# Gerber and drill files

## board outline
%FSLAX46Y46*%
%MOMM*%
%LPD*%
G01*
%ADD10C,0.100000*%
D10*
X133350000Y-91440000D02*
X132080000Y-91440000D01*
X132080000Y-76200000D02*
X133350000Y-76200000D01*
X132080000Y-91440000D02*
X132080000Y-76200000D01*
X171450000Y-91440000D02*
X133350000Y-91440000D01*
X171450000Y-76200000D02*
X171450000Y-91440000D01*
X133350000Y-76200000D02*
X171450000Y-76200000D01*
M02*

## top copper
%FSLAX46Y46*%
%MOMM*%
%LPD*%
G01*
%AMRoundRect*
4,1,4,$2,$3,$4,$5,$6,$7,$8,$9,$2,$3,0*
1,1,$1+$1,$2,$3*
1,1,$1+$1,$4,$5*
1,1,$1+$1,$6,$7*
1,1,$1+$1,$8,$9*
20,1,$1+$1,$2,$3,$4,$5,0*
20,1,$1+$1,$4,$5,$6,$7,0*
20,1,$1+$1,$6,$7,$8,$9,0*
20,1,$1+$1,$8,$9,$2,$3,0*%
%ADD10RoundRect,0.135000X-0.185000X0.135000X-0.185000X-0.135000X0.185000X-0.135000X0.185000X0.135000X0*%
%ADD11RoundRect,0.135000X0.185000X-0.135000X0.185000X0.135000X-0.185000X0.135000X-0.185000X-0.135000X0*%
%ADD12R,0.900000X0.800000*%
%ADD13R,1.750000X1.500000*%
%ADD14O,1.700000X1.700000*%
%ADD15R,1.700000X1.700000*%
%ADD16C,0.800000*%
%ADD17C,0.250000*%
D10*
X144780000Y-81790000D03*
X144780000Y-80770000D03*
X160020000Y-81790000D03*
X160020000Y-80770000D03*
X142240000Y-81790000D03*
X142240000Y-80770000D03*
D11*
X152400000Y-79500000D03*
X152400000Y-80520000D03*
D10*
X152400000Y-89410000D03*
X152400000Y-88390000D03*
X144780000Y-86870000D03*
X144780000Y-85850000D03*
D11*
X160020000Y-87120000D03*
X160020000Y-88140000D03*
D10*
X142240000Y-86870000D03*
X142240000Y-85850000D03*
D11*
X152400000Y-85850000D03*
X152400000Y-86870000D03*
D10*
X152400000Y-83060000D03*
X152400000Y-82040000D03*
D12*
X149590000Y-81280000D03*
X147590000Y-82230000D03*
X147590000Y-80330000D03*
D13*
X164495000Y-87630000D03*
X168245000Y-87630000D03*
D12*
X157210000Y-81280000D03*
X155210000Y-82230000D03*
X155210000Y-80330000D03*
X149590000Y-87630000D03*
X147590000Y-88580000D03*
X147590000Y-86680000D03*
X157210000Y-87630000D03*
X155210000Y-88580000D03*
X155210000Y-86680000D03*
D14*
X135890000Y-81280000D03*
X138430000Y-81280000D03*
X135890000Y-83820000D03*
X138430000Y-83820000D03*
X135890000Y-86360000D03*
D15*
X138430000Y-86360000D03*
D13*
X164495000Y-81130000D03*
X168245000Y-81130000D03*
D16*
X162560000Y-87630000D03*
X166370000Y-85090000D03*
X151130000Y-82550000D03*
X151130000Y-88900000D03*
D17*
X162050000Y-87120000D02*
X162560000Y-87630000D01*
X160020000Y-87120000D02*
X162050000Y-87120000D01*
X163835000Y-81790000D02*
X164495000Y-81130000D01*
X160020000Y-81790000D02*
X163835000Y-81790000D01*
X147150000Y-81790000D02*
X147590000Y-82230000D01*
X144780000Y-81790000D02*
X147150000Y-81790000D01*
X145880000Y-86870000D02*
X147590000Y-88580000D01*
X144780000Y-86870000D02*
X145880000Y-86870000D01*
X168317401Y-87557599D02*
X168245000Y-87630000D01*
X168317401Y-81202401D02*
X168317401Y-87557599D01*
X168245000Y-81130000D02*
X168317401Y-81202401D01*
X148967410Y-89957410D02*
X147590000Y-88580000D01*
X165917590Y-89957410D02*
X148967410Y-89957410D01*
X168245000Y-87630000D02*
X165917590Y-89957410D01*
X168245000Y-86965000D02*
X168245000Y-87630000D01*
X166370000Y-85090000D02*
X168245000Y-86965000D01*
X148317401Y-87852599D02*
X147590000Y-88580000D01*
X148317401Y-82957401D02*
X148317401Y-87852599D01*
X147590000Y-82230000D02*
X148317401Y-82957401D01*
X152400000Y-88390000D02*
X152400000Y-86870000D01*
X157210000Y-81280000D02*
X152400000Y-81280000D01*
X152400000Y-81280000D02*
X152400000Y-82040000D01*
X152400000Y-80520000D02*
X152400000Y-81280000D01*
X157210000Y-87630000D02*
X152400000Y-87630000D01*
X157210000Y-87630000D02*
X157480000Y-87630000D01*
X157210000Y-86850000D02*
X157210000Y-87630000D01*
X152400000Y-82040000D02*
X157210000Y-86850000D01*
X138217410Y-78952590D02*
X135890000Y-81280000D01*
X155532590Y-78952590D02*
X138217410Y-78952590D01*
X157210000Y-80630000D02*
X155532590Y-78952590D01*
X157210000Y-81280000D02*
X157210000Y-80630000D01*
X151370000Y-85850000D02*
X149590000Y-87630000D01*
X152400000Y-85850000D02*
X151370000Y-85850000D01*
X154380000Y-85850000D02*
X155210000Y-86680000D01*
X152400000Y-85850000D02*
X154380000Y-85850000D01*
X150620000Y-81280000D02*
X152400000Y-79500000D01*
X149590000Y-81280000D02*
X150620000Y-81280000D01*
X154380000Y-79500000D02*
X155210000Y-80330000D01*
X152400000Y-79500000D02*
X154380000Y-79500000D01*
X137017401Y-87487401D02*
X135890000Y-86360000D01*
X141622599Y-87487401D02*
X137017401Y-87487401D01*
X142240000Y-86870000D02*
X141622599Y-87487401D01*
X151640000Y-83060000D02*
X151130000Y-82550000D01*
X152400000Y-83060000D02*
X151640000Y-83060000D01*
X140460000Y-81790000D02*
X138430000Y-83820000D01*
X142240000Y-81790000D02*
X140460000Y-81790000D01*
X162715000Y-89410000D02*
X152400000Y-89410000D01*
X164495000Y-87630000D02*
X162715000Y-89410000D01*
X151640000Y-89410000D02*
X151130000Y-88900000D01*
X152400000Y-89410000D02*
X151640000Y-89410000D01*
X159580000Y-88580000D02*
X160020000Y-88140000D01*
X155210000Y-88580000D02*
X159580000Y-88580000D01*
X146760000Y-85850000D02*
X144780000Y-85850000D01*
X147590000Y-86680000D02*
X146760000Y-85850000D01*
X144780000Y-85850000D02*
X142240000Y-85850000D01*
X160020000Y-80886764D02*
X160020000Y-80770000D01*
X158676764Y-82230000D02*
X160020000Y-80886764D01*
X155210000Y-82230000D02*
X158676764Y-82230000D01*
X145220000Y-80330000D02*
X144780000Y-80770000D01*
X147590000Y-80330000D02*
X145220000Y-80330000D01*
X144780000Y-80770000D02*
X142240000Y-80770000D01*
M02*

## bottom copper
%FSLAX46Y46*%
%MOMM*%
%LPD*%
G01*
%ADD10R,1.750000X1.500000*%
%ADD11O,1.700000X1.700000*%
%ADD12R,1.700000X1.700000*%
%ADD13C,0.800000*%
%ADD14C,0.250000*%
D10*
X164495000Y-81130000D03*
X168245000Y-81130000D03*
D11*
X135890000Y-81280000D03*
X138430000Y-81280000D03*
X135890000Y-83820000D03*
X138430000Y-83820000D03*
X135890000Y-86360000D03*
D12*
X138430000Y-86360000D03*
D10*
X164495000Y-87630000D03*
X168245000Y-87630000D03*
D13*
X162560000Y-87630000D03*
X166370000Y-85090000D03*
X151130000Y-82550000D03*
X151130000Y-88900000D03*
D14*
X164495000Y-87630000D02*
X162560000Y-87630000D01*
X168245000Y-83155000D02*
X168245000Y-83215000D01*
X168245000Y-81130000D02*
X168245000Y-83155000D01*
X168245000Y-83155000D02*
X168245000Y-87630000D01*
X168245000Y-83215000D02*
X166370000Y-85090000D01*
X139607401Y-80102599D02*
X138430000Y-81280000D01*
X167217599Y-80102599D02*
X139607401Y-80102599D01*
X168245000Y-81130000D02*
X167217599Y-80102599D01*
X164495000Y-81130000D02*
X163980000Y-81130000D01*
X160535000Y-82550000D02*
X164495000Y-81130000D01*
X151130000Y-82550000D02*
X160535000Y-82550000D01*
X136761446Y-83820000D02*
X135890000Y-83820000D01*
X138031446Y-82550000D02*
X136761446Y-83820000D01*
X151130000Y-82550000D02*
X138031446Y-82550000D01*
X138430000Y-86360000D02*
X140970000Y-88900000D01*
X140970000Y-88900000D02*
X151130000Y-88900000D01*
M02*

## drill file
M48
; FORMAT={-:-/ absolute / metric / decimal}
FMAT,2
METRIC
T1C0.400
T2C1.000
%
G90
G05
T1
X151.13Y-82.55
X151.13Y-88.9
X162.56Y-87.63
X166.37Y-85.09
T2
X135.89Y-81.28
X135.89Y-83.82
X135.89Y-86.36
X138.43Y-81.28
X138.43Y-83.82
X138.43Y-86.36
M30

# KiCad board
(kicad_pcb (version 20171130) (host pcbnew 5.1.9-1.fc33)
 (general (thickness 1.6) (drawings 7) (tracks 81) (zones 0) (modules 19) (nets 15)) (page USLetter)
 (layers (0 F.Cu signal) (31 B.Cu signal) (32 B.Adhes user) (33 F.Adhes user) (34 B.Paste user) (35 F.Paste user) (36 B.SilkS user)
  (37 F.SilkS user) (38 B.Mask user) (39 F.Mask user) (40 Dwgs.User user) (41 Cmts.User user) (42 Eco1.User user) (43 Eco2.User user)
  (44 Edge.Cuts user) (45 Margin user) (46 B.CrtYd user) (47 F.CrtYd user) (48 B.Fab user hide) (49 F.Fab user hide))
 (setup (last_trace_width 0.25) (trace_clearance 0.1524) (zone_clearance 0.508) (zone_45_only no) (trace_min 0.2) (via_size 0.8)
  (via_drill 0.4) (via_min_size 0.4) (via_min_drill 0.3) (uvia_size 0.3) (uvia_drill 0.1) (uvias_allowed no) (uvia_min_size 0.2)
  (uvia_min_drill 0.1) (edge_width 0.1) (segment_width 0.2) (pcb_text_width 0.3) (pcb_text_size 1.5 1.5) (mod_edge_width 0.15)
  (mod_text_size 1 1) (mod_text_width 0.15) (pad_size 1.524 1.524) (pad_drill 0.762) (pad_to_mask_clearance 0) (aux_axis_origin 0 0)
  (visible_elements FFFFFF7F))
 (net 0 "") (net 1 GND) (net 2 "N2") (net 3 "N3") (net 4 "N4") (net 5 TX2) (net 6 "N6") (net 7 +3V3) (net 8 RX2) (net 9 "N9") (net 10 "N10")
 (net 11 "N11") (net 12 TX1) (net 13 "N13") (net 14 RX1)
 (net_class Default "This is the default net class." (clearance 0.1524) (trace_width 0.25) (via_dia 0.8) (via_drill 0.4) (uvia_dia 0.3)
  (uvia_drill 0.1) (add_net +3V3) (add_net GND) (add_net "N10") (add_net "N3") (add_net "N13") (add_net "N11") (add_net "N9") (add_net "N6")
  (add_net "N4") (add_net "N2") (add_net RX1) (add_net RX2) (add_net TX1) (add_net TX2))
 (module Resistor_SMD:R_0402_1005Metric (layer F.Cu) (at 144.78 81.28 270)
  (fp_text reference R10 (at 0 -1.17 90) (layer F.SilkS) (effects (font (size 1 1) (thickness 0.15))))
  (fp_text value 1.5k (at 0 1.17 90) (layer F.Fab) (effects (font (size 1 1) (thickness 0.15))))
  (pad 2 smd roundrect (at 0.51 0 270) (size 0.54 0.64) (layers F.Cu F.Paste F.Mask) (roundrect_rratio 0.25) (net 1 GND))
  (pad 1 smd roundrect (at -0.51 0 270) (size 0.54 0.64) (layers F.Cu F.Paste F.Mask) (roundrect_rratio 0.25) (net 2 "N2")))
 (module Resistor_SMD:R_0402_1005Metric (layer F.Cu) (at 160.02 81.28 270)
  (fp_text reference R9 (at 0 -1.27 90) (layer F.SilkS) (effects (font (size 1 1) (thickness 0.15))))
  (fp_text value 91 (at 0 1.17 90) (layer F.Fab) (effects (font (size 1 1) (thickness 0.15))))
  (pad 2 smd roundrect (at 0.51 0 270) (size 0.54 0.64) (layers F.Cu F.Paste F.Mask) (roundrect_rratio 0.25) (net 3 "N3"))
  (pad 1 smd roundrect (at -0.51 0 270) (size 0.54 0.64) (layers F.Cu F.Paste F.Mask) (roundrect_rratio 0.25) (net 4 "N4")))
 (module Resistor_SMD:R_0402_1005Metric (layer F.Cu) (at 142.24 81.28 270)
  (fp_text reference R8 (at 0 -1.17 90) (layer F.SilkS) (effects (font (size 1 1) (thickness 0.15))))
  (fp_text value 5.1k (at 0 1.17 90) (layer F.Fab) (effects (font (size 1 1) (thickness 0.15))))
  (pad 2 smd roundrect (at 0.51 0 270) (size 0.54 0.64) (layers F.Cu F.Paste F.Mask) (roundrect_rratio 0.25) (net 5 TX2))
  (pad 1 smd roundrect (at -0.51 0 270) (size 0.54 0.64) (layers F.Cu F.Paste F.Mask) (roundrect_rratio 0.25) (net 2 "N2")))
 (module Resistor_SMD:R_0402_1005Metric (layer F.Cu) (at 152.4 80.01 90)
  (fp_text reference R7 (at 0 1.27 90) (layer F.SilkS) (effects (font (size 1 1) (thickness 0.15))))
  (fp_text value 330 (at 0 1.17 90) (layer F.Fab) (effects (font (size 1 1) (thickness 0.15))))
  (pad 2 smd roundrect (at 0.51 0 90) (size 0.54 0.64) (layers F.Cu F.Paste F.Mask) (roundrect_rratio 0.25) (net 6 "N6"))
  (pad 1 smd roundrect (at -0.51 0 90) (size 0.54 0.64) (layers F.Cu F.Paste F.Mask) (roundrect_rratio 0.25) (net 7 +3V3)))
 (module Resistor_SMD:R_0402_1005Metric (layer F.Cu) (at 152.4 88.9 270)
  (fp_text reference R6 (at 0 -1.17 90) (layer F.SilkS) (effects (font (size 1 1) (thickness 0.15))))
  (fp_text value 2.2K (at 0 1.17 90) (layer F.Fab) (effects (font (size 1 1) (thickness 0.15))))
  (pad 2 smd roundrect (at 0.51 0 270) (size 0.54 0.64) (layers F.Cu F.Paste F.Mask) (roundrect_rratio 0.25) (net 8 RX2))
  (pad 1 smd roundrect (at -0.51 0 270) (size 0.54 0.64) (layers F.Cu F.Paste F.Mask) (roundrect_rratio 0.25) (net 7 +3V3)))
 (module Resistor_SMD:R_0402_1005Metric (layer F.Cu) (at 144.78 86.36 270)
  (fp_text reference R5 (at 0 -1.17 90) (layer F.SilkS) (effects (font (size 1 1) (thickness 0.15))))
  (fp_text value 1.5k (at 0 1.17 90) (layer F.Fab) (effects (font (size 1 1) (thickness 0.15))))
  (pad 2 smd roundrect (at 0.51 0 270) (size 0.54 0.64) (layers F.Cu F.Paste F.Mask) (roundrect_rratio 0.25) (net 1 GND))
  (pad 1 smd roundrect (at -0.51 0 270) (size 0.54 0.64) (layers F.Cu F.Paste F.Mask) (roundrect_rratio 0.25) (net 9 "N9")))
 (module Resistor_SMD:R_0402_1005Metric (layer F.Cu) (at 160.02 87.63 90)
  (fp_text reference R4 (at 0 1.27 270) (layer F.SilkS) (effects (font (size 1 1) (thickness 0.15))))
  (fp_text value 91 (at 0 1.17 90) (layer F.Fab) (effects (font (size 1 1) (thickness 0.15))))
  (pad 2 smd roundrect (at 0.51 0 90) (size 0.54 0.64) (layers F.Cu F.Paste F.Mask) (roundrect_rratio 0.25) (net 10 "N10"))
  (pad 1 smd roundrect (at -0.51 0 90) (size 0.54 0.64) (layers F.Cu F.Paste F.Mask) (roundrect_rratio 0.25) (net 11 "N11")))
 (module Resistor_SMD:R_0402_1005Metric (layer F.Cu) (at 142.24 86.36 270)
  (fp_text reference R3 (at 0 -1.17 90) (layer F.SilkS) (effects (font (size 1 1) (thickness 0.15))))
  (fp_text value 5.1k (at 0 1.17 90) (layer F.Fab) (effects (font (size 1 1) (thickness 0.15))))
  (pad 2 smd roundrect (at 0.51 0 270) (size 0.54 0.64) (layers F.Cu F.Paste F.Mask) (roundrect_rratio 0.25) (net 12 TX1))
  (pad 1 smd roundrect (at -0.51 0 270) (size 0.54 0.64) (layers F.Cu F.Paste F.Mask) (roundrect_rratio 0.25) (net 9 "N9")))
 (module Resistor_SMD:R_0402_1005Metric (layer F.Cu) (at 152.4 86.36 90)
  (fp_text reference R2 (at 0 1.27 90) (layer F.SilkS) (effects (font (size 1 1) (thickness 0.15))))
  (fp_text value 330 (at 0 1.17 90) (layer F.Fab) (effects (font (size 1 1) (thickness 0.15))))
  (pad 2 smd roundrect (at 0.51 0 90) (size 0.54 0.64) (layers F.Cu F.Paste F.Mask) (roundrect_rratio 0.25) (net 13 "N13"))
  (pad 1 smd roundrect (at -0.51 0 90) (size 0.54 0.64) (layers F.Cu F.Paste F.Mask) (roundrect_rratio 0.25) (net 7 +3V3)))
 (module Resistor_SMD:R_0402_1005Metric (layer F.Cu) (at 152.4 82.55 270)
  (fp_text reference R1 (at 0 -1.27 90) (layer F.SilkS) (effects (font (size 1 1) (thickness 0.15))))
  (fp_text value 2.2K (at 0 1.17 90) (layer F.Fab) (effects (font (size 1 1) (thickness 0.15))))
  (pad 2 smd roundrect (at 0.51 0 270) (size 0.54 0.64) (layers F.Cu F.Paste F.Mask) (roundrect_rratio 0.25) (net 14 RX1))
  (pad 1 smd roundrect (at -0.51 0 270) (size 0.54 0.64) (layers F.Cu F.Paste F.Mask) (roundrect_rratio 0.25) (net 7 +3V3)))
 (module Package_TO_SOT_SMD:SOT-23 (layer F.Cu) (at 148.59 81.28)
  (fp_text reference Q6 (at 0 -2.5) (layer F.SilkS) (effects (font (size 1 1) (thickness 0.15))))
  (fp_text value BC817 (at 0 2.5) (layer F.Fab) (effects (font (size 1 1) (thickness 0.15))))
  (pad 3 smd rect (at 1 0) (size 0.9 0.8) (layers F.Cu F.Paste F.Mask) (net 6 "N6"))
  (pad 2 smd rect (at -1 0.95) (size 0.9 0.8) (layers F.Cu F.Paste F.Mask) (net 1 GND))
  (pad 1 smd rect (at -1 -0.95) (size 0.9 0.8) (layers F.Cu F.Paste F.Mask) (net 2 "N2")))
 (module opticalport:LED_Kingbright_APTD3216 (layer F.Cu) (at 166.37 87.63 180)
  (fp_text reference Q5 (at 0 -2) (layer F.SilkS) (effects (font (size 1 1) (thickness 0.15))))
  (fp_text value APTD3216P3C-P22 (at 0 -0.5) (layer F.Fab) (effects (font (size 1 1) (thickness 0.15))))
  (pad 2 smd rect (at 1.875 0 180) (size 1.75 1.5) (layers F.Cu F.Paste F.Mask) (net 8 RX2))
  (pad 1 smd rect (at -1.875 0 180) (size 1.75 1.5) (layers F.Cu F.Paste F.Mask) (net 1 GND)))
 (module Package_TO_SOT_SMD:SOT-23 (layer F.Cu) (at 156.21 81.28)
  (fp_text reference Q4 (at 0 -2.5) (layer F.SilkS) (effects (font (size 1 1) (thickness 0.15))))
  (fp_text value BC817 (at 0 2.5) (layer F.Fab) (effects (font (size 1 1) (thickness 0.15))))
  (pad 3 smd rect (at 1 0) (size 0.9 0.8) (layers F.Cu F.Paste F.Mask) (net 7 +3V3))
  (pad 2 smd rect (at -1 0.95) (size 0.9 0.8) (layers F.Cu F.Paste F.Mask) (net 4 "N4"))
  (pad 1 smd rect (at -1 -0.95) (size 0.9 0.8) (layers F.Cu F.Paste F.Mask) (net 6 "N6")))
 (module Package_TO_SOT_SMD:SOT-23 (layer F.Cu) (at 148.59 87.63)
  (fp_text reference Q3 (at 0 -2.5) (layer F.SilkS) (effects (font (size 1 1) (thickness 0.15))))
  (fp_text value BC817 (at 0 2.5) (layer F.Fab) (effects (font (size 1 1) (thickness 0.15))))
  (pad 3 smd rect (at 1 0) (size 0.9 0.8) (layers F.Cu F.Paste F.Mask) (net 13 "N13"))
  (pad 2 smd rect (at -1 0.95) (size 0.9 0.8) (layers F.Cu F.Paste F.Mask) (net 1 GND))
  (pad 1 smd rect (at -1 -0.95) (size 0.9 0.8) (layers F.Cu F.Paste F.Mask) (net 9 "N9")))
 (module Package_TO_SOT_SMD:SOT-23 (layer F.Cu) (at 156.21 87.63)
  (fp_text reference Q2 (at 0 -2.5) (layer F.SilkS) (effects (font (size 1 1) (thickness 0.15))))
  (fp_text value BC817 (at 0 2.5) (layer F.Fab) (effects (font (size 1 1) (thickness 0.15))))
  (pad 3 smd rect (at 1 0) (size 0.9 0.8) (layers F.Cu F.Paste F.Mask) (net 7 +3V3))
  (pad 2 smd rect (at -1 0.95) (size 0.9 0.8) (layers F.Cu F.Paste F.Mask) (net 11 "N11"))
  (pad 1 smd rect (at -1 -0.95) (size 0.9 0.8) (layers F.Cu F.Paste F.Mask) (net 13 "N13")))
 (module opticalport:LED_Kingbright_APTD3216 (layer B.Cu) (at 166.37 81.13 180)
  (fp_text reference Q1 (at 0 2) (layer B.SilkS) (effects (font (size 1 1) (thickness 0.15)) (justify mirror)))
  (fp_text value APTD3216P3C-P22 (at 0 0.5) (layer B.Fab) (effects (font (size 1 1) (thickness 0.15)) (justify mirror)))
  (pad 2 smd rect (at 1.875 0 180) (size 1.75 1.5) (layers B.Cu B.Paste B.Mask) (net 14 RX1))
  (pad 1 smd rect (at -1.875 0 180) (size 1.75 1.5) (layers B.Cu B.Paste B.Mask) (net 1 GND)))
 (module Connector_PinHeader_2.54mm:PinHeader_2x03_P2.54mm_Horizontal (layer F.Cu) (at 138.43 86.36 180)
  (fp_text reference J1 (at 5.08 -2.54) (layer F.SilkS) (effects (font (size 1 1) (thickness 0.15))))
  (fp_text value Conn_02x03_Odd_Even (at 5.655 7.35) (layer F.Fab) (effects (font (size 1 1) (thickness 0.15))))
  (pad 6 thru_hole oval (at 2.54 5.08 180) (size 1.7 1.7) (drill 1) (layers *.Cu *.Mask) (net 7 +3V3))
  (pad 5 thru_hole oval (at 0 5.08 180) (size 1.7 1.7) (drill 1) (layers *.Cu *.Mask) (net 1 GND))
  (pad 4 thru_hole oval (at 2.54 2.54 180) (size 1.7 1.7) (drill 1) (layers *.Cu *.Mask) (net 14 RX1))
  (pad 3 thru_hole oval (at 0 2.54 180) (size 1.7 1.7) (drill 1) (layers *.Cu *.Mask) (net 5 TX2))
  (pad 2 thru_hole oval (at 2.54 0 180) (size 1.7 1.7) (drill 1) (layers *.Cu *.Mask) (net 12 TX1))
  (pad 1 thru_hole rect (at 0 0 180) (size 1.7 1.7) (drill 1) (layers *.Cu *.Mask) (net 8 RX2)))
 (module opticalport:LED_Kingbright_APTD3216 (layer F.Cu) (at 166.37 81.13 180)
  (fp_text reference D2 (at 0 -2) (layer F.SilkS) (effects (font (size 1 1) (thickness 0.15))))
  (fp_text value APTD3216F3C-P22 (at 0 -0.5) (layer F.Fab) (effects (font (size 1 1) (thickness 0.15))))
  (pad 2 smd rect (at 1.875 0 180) (size 1.75 1.5) (layers F.Cu F.Paste F.Mask) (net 3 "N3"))
  (pad 1 smd rect (at -1.875 0 180) (size 1.75 1.5) (layers F.Cu F.Paste F.Mask) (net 1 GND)))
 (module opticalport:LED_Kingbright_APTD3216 (layer B.Cu) (at 166.37 87.63 180)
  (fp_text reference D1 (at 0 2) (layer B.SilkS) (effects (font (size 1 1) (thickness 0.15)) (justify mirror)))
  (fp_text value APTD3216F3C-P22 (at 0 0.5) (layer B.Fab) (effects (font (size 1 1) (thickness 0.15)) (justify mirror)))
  (pad 2 smd rect (at 1.875 0 180) (size 1.75 1.5) (layers B.Cu B.Paste B.Mask) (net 10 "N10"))
  (pad 1 smd rect (at -1.875 0 180) (size 1.75 1.5) (layers B.Cu B.Paste B.Mask) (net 1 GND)))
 (gr_line (start 133.35 91.44) (end 132.08 91.44) (layer Edge.Cuts) (width 0.1))
 (gr_line (start 132.08 76.2) (end 133.35 76.2) (layer Edge.Cuts) (width 0.1))
 (gr_line (start 132.08 91.44) (end 132.08 76.2) (layer Edge.Cuts) (width 0.1))
 (gr_line (start 171.45 91.44) (end 133.35 91.44) (layer Edge.Cuts) (width 0.1))
 (gr_line (start 171.45 76.2) (end 171.45 91.44) (layer Edge.Cuts) (width 0.1))
 (gr_line (start 133.35 76.2) (end 171.45 76.2) (layer Edge.Cuts) (width 0.1))
 (segment (start 164.495 87.63) (end 162.56 87.63) (width 0.25) (layer B.Cu) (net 10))
 (via (at 162.56 87.63) (size 0.8) (drill 0.4) (layers F.Cu B.Cu) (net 10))
 (segment (start 162.05 87.12) (end 162.56 87.63) (width 0.25) (layer F.Cu) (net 10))
 (segment (start 160.02 87.12) (end 162.05 87.12) (width 0.25) (layer F.Cu) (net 10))
 (segment (start 163.835 81.79) (end 164.495 81.13) (width 0.25) (layer F.Cu) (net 3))
 (segment (start 160.02 81.79) (end 163.835 81.79) (width 0.25) (layer F.Cu) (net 3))
 (segment (start 147.15 81.79) (end 147.59 82.23) (width 0.25) (layer F.Cu) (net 1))
 (segment (start 144.78 81.79) (end 147.15 81.79) (width 0.25) (layer F.Cu) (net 1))
 (segment (start 145.88 86.87) (end 147.59 88.58) (width 0.25) (layer F.Cu) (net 1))
 (segment (start 144.78 86.87) (end 145.88 86.87) (width 0.25) (layer F.Cu) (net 1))
 (segment (start 168.317401 87.557599) (end 168.245 87.63) (width 0.25) (layer F.Cu) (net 1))
 (segment (start 168.317401 81.202401) (end 168.317401 87.557599) (width 0.25) (layer F.Cu) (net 1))
 (segment (start 168.245 81.13) (end 168.317401 81.202401) (width 0.25) (layer F.Cu) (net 1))
 (segment (start 148.96741 89.95741) (end 147.59 88.58) (width 0.25) (layer F.Cu) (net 1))
 (segment (start 165.91759 89.95741) (end 148.96741 89.95741) (width 0.25) (layer F.Cu) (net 1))
 (segment (start 168.245 87.63) (end 165.91759 89.95741) (width 0.25) (layer F.Cu) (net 1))
 (segment (start 168.245 83.155) (end 168.245 83.215) (width 0.25) (layer B.Cu) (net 1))
 (segment (start 168.245 81.13) (end 168.245 83.155) (width 0.25) (layer B.Cu) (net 1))
 (segment (start 168.245 83.155) (end 168.245 87.63) (width 0.25) (layer B.Cu) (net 1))
 (via (at 166.37 85.09) (size 0.8) (drill 0.4) (layers F.Cu B.Cu) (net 1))
 (segment (start 168.245 83.215) (end 166.37 85.09) (width 0.25) (layer B.Cu) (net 1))
 (segment (start 168.245 86.965) (end 168.245 87.63) (width 0.25) (layer F.Cu) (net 1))
 (segment (start 166.37 85.09) (end 168.245 86.965) (width 0.25) (layer F.Cu) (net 1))
 (segment (start 148.317401 87.852599) (end 147.59 88.58) (width 0.25) (layer F.Cu) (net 1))
 (segment (start 148.317401 82.957401) (end 148.317401 87.852599) (width 0.25) (layer F.Cu) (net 1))
 (segment (start 147.59 82.23) (end 148.317401 82.957401) (width 0.25) (layer F.Cu) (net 1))
 (segment (start 139.607401 80.102599) (end 138.43 81.28) (width 0.25) (layer B.Cu) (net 1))
 (segment (start 167.217599 80.102599) (end 139.607401 80.102599) (width 0.25) (layer B.Cu) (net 1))
 (segment (start 168.245 81.13) (end 167.217599 80.102599) (width 0.25) (layer B.Cu) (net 1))
 (segment (start 152.4 88.39) (end 152.4 86.87) (width 0.25) (layer F.Cu) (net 7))
 (segment (start 157.21 81.28) (end 152.4 81.28) (width 0.25) (layer F.Cu) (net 7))
 (segment (start 152.4 81.28) (end 152.4 82.04) (width 0.25) (layer F.Cu) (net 7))
 (segment (start 152.4 80.52) (end 152.4 81.28) (width 0.25) (layer F.Cu) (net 7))
 (segment (start 157.21 87.63) (end 152.4 87.63) (width 0.25) (layer F.Cu) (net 7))
 (segment (start 157.21 87.63) (end 157.48 87.63) (width 0.25) (layer F.Cu) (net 7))
 (segment (start 157.21 86.85) (end 157.21 87.63) (width 0.25) (layer F.Cu) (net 7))
 (segment (start 152.4 82.04) (end 157.21 86.85) (width 0.25) (layer F.Cu) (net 7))
 (segment (start 138.21741 78.95259) (end 135.89 81.28) (width 0.25) (layer F.Cu) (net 7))
 (segment (start 155.53259 78.95259) (end 138.21741 78.95259) (width 0.25) (layer F.Cu) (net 7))
 (segment (start 157.21 80.63) (end 155.53259 78.95259) (width 0.25) (layer F.Cu) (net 7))
 (segment (start 157.21 81.28) (end 157.21 80.63) (width 0.25) (layer F.Cu) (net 7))
 (segment (start 151.37 85.85) (end 149.59 87.63) (width 0.25) (layer F.Cu) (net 13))
 (segment (start 152.4 85.85) (end 151.37 85.85) (width 0.25) (layer F.Cu) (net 13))
 (segment (start 154.38 85.85) (end 155.21 86.68) (width 0.25) (layer F.Cu) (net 13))
 (segment (start 152.4 85.85) (end 154.38 85.85) (width 0.25) (layer F.Cu) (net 13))
 (segment (start 150.62 81.28) (end 152.4 79.5) (width 0.25) (layer F.Cu) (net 6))
 (segment (start 149.59 81.28) (end 150.62 81.28) (width 0.25) (layer F.Cu) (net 6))
 (segment (start 154.38 79.5) (end 155.21 80.33) (width 0.25) (layer F.Cu) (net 6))
 (segment (start 152.4 79.5) (end 154.38 79.5) (width 0.25) (layer F.Cu) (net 6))
 (segment (start 137.017401 87.487401) (end 135.89 86.36) (width 0.25) (layer F.Cu) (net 12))
 (segment (start 141.622599 87.487401) (end 137.017401 87.487401) (width 0.25) (layer F.Cu) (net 12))
 (segment (start 142.24 86.87) (end 141.622599 87.487401) (width 0.25) (layer F.Cu) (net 12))
 (segment (start 164.495 81.13) (end 163.98 81.13) (width 0.25) (layer B.Cu) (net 14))
 (via (at 151.13 82.55) (size 0.8) (drill 0.4) (layers F.Cu B.Cu) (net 14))
 (segment (start 160.535 82.55) (end 164.495 81.13) (width 0.25) (layer B.Cu) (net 14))
 (segment (start 151.13 82.55) (end 160.535 82.55) (width 0.25) (layer B.Cu) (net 14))
 (segment (start 136.761446 83.82) (end 135.89 83.82) (width 0.25) (layer B.Cu) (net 14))
 (segment (start 138.031446 82.55) (end 136.761446 83.82) (width 0.25) (layer B.Cu) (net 14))
 (segment (start 151.13 82.55) (end 138.031446 82.55) (width 0.25) (layer B.Cu) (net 14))
 (segment (start 151.64 83.06) (end 151.13 82.55) (width 0.25) (layer F.Cu) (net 14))
 (segment (start 152.4 83.06) (end 151.64 83.06) (width 0.25) (layer F.Cu) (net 14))
 (segment (start 140.46 81.79) (end 138.43 83.82) (width 0.25) (layer F.Cu) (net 5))
 (segment (start 142.24 81.79) (end 140.46 81.79) (width 0.25) (layer F.Cu) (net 5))
 (segment (start 162.715 89.41) (end 152.4 89.41) (width 0.25) (layer F.Cu) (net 8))
 (segment (start 164.495 87.63) (end 162.715 89.41) (width 0.25) (layer F.Cu) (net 8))
 (segment (start 138.43 86.36) (end 140.97 88.9) (width 0.25) (layer B.Cu) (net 8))
 (via (at 151.13 88.9) (size 0.8) (drill 0.4) (layers F.Cu B.Cu) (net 8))
 (segment (start 140.97 88.9) (end 151.13 88.9) (width 0.25) (layer B.Cu) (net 8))
 (segment (start 151.64 89.41) (end 151.13 88.9) (width 0.25) (layer F.Cu) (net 8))
 (segment (start 152.4 89.41) (end 151.64 89.41) (width 0.25) (layer F.Cu) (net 8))
 (segment (start 159.58 88.58) (end 160.02 88.14) (width 0.25) (layer F.Cu) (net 11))
 (segment (start 155.21 88.58) (end 159.58 88.58) (width 0.25) (layer F.Cu) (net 11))
 (segment (start 146.76 85.85) (end 144.78 85.85) (width 0.25) (layer F.Cu) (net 9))
 (segment (start 147.59 86.68) (end 146.76 85.85) (width 0.25) (layer F.Cu) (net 9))
 (segment (start 144.78 85.85) (end 142.24 85.85) (width 0.25) (layer F.Cu) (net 9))
 (segment (start 160.02 80.886764) (end 160.02 80.77) (width 0.25) (layer F.Cu) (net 4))
 (segment (start 158.676764 82.23) (end 160.02 80.886764) (width 0.25) (layer F.Cu) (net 4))
 (segment (start 155.21 82.23) (end 158.676764 82.23) (width 0.25) (layer F.Cu) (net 4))
 (segment (start 145.22 80.33) (end 144.78 80.77) (width 0.25) (layer F.Cu) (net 2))
 (segment (start 147.59 80.33) (end 145.22 80.33) (width 0.25) (layer F.Cu) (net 2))
 (segment (start 144.78 80.77) (end 142.24 80.77) (width 0.25) (layer F.Cu) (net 2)))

